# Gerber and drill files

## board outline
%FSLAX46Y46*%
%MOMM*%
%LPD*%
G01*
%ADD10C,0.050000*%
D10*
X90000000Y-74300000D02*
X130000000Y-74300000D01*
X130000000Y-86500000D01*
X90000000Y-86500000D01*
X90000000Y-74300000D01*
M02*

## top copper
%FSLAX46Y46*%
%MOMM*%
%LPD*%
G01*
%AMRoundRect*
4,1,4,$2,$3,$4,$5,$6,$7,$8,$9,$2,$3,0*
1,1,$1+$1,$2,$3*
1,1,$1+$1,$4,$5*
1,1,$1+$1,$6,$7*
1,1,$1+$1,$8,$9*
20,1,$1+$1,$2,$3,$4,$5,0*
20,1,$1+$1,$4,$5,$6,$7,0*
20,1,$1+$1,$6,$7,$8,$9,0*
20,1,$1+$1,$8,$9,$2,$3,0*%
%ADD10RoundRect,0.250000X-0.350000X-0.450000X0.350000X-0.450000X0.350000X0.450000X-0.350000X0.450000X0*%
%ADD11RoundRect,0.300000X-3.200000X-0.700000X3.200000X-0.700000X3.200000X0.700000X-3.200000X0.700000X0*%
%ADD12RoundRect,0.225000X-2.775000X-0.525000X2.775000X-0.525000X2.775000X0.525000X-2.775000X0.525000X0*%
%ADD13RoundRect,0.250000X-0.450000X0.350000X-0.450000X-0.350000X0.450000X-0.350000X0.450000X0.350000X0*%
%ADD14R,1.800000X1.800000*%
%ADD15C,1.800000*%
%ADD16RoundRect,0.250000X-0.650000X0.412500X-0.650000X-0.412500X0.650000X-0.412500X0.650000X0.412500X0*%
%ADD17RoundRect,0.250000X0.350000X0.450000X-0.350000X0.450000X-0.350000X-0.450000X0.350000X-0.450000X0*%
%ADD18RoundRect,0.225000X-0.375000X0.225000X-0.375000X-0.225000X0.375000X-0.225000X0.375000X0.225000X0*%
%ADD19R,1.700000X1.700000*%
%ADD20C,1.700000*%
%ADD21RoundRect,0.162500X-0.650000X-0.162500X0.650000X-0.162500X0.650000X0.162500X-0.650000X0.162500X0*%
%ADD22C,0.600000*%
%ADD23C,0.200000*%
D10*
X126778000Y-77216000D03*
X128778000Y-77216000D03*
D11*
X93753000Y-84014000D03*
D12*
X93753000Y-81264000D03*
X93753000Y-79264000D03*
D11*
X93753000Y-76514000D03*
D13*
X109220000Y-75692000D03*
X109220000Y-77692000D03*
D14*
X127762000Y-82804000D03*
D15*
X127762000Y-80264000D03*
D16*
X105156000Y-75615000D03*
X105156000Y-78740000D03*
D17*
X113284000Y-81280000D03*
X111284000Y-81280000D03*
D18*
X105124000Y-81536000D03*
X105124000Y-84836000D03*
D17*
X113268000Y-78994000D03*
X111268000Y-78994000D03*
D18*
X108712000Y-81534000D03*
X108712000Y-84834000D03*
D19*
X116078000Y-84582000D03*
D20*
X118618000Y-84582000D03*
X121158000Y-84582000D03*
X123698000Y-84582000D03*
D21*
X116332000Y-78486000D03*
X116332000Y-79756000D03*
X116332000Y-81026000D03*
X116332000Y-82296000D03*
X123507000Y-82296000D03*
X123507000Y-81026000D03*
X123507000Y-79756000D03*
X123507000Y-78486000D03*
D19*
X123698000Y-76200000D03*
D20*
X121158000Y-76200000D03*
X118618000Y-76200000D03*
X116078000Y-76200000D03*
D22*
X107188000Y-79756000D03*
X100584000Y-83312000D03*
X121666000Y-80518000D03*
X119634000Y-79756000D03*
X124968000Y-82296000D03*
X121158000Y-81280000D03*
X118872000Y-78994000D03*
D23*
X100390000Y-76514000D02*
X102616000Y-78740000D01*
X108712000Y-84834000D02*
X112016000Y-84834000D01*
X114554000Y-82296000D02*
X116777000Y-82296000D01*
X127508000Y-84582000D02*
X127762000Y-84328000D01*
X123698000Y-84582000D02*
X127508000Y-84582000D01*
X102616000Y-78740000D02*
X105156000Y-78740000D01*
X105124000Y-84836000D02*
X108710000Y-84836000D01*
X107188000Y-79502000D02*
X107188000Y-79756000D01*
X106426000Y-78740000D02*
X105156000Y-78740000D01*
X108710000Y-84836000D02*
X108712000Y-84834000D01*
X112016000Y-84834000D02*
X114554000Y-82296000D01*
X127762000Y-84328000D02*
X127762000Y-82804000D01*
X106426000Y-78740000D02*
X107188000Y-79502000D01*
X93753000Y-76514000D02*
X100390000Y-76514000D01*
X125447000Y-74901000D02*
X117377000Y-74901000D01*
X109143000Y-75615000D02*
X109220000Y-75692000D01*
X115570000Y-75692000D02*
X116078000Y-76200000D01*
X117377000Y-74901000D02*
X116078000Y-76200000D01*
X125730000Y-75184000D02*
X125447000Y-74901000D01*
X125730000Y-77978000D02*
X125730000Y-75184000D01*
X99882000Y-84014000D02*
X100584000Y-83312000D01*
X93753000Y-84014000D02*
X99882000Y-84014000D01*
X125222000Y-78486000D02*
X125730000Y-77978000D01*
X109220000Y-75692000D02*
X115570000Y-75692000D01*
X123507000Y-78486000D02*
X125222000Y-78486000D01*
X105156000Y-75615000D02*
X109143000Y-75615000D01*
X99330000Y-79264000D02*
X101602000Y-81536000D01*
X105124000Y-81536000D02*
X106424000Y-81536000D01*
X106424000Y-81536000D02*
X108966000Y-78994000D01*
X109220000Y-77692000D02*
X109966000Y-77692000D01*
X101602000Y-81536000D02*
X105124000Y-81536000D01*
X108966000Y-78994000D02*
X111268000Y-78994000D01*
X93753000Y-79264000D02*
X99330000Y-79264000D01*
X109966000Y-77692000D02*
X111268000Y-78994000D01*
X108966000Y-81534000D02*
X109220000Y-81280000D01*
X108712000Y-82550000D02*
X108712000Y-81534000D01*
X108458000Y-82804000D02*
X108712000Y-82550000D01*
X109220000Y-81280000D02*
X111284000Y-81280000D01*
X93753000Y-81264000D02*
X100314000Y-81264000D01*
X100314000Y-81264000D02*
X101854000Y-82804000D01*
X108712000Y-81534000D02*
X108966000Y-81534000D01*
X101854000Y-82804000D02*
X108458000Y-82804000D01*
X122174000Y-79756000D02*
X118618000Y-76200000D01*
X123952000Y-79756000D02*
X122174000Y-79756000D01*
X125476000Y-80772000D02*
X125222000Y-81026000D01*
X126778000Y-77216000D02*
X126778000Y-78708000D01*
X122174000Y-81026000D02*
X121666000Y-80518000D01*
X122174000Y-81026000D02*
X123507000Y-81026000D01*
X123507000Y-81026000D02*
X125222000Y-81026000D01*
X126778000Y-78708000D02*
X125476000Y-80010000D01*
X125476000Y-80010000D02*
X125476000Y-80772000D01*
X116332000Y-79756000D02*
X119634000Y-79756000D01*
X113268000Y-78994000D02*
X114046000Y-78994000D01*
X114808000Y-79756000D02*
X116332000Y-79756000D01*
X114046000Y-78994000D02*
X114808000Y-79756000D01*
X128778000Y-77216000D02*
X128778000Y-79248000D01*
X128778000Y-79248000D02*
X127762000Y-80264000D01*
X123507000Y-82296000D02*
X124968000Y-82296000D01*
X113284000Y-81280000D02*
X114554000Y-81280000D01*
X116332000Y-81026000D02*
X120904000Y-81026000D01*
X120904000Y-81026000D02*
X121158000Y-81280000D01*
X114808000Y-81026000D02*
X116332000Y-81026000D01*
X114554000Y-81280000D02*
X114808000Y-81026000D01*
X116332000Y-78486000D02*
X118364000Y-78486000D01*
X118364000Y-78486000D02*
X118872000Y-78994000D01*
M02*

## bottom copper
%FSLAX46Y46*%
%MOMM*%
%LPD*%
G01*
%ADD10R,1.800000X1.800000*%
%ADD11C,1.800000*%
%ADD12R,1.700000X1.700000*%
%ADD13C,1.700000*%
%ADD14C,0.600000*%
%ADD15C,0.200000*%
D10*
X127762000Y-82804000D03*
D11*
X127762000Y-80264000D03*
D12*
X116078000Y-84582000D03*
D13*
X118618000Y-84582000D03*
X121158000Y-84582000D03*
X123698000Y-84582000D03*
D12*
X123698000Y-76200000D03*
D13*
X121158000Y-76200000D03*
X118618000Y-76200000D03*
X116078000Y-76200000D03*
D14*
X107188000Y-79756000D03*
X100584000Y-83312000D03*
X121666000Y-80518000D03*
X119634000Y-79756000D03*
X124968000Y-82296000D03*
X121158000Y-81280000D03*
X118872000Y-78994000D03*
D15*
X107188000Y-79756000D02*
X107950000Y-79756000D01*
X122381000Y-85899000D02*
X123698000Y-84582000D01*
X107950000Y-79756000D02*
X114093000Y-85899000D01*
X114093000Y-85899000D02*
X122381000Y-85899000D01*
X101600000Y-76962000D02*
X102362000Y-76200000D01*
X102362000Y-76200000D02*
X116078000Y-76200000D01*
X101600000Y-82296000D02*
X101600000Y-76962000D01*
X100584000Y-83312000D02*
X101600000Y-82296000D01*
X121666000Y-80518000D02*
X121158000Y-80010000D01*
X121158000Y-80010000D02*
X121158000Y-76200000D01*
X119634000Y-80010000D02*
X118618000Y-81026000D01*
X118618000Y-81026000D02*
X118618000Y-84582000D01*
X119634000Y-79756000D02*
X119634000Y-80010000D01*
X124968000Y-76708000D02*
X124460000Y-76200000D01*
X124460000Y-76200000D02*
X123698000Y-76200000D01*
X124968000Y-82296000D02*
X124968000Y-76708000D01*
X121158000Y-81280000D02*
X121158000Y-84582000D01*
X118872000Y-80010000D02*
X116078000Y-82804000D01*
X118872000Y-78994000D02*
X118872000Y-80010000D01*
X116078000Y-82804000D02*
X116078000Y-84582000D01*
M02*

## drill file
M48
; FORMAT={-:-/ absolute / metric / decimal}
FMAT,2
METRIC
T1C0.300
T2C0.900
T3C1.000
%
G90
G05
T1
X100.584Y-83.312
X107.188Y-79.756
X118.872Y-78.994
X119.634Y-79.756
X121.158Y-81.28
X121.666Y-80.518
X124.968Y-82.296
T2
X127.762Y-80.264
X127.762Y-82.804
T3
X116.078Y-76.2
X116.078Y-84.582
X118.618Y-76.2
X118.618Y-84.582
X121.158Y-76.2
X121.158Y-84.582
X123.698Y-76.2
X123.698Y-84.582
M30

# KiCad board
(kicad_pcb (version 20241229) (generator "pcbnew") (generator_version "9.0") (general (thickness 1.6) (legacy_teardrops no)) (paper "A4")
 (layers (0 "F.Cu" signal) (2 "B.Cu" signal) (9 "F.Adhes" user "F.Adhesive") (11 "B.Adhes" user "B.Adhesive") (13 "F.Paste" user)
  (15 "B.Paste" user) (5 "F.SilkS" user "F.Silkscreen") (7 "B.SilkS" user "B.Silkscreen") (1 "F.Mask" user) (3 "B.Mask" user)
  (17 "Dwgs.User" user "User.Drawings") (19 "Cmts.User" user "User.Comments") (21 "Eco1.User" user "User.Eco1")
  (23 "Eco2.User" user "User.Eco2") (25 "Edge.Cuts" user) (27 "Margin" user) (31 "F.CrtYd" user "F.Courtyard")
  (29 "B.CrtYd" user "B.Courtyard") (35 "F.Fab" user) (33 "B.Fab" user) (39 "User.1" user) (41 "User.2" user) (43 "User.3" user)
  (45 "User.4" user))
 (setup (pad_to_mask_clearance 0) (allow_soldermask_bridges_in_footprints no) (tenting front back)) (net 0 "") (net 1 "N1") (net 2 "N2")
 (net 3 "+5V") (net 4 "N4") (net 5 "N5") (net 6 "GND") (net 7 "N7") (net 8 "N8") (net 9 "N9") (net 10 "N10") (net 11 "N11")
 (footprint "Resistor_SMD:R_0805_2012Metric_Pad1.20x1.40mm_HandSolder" (layer "F.Cu") (at 127.778 77.216)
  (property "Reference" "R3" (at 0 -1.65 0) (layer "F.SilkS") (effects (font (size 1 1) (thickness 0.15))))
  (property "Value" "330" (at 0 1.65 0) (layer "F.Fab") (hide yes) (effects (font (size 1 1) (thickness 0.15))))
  (pad "1" smd roundrect (at -1 0) (size 1.2 1.4) (layers "F.Cu" "F.Mask" "F.Paste") (roundrect_rratio 0.208333) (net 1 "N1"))
  (pad "2" smd roundrect (at 1 0) (size 1.2 1.4) (layers "F.Cu" "F.Mask" "F.Paste") (roundrect_rratio 0.208333) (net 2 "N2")))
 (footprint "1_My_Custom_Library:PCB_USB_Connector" (layer "F.Cu") (at 93.753 80.264)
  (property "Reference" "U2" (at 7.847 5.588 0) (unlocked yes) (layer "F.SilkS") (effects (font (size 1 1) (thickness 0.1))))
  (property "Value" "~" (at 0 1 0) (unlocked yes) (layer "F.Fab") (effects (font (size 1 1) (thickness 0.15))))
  (pad "1" smd roundrect (at 0 3.75) (size 7 2) (layers "F.Cu" "F.Mask" "F.Paste") (roundrect_rratio 0.15) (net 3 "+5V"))
  (pad "2" smd roundrect (at 0 1) (size 6 1.5) (layers "F.Cu" "F.Mask" "F.Paste") (roundrect_rratio 0.15) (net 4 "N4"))
  (pad "3" smd roundrect (at 0 -1) (size 6 1.5) (layers "F.Cu" "F.Mask" "F.Paste") (roundrect_rratio 0.15) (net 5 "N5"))
  (pad "4" smd roundrect (at 0 -3.75) (size 7 2) (layers "F.Cu" "F.Mask" "F.Paste") (roundrect_rratio 0.15) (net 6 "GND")))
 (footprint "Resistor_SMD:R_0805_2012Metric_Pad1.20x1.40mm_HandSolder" (layer "F.Cu") (at 109.22 76.692 -90)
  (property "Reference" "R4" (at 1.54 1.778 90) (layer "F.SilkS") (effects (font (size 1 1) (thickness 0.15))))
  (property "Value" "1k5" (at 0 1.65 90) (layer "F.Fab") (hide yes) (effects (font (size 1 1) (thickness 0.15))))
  (pad "1" smd roundrect (at -1 0 270) (size 1.2 1.4) (layers "F.Cu" "F.Mask" "F.Paste") (roundrect_rratio 0.208333) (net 3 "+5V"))
  (pad "2" smd roundrect (at 1 0 270) (size 1.2 1.4) (layers "F.Cu" "F.Mask" "F.Paste") (roundrect_rratio 0.208333) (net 5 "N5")))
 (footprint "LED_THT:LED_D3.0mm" (layer "F.Cu") (at 127.762 82.804 90)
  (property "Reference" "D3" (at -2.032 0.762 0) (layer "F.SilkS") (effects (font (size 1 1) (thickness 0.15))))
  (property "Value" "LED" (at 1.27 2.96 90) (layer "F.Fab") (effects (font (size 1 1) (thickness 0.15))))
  (pad "1" thru_hole rect (at 0 0 90) (size 1.8 1.8) (drill 0.9) (layers "*.Cu" "*.Mask") (remove_unused_layers no) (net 6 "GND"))
  (pad "2" thru_hole circle (at 2.54 0 90) (size 1.8 1.8) (drill 0.9) (layers "*.Cu" "*.Mask") (remove_unused_layers no) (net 2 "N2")))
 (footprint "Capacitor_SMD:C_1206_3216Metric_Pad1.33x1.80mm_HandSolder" (layer "F.Cu") (at 105.156 77.1775 -90)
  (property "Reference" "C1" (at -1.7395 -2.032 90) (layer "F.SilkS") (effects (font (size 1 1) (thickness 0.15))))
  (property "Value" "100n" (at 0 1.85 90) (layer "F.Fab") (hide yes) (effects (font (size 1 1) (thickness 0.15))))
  (pad "1" smd roundrect (at -1.5625 0 270) (size 1.325 1.8) (layers "F.Cu" "F.Mask" "F.Paste") (roundrect_rratio 0.188679) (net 3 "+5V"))
  (pad "2" smd roundrect (at 1.5625 0 270) (size 1.325 1.8) (layers "F.Cu" "F.Mask" "F.Paste") (roundrect_rratio 0.188679) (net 6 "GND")))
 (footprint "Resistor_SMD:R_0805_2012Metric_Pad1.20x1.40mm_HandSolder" (layer "F.Cu") (at 112.284 81.28 180)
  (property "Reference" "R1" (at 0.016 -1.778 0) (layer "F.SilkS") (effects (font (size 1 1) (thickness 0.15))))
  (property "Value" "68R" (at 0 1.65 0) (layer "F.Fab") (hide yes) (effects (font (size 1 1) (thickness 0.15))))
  (pad "1" smd roundrect (at -1 0 180) (size 1.2 1.4) (layers "F.Cu" "F.Mask" "F.Paste") (roundrect_rratio 0.208333) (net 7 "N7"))
  (pad "2" smd roundrect (at 1 0 180) (size 1.2 1.4) (layers "F.Cu" "F.Mask" "F.Paste") (roundrect_rratio 0.208333) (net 4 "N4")))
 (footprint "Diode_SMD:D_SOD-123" (layer "F.Cu") (at 105.124 83.186 -90)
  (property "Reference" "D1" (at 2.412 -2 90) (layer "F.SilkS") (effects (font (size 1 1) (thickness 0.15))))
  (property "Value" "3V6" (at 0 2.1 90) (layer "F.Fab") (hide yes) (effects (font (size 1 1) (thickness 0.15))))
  (pad "1" smd roundrect (at -1.65 0 270) (size 0.9 1.2) (layers "F.Cu" "F.Mask" "F.Paste") (roundrect_rratio 0.25) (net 5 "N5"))
  (pad "2" smd roundrect (at 1.65 0 270) (size 0.9 1.2) (layers "F.Cu" "F.Mask" "F.Paste") (roundrect_rratio 0.25) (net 6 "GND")))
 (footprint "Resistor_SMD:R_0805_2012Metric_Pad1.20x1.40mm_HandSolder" (layer "F.Cu") (at 112.268 78.994 180)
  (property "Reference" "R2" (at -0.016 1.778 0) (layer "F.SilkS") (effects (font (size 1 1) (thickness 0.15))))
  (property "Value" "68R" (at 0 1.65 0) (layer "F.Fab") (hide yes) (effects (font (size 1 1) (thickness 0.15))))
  (pad "1" smd roundrect (at -1 0 180) (size 1.2 1.4) (layers "F.Cu" "F.Mask" "F.Paste") (roundrect_rratio 0.208333) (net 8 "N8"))
  (pad "2" smd roundrect (at 1 0 180) (size 1.2 1.4) (layers "F.Cu" "F.Mask" "F.Paste") (roundrect_rratio 0.208333) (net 5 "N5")))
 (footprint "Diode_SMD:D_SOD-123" (layer "F.Cu") (at 108.712 83.184 -90)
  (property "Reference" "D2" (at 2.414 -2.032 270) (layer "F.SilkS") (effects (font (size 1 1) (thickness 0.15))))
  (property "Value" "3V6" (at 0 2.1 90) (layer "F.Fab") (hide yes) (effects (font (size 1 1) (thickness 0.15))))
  (pad "1" smd roundrect (at -1.65 0 270) (size 0.9 1.2) (layers "F.Cu" "F.Mask" "F.Paste") (roundrect_rratio 0.25) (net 4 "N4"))
  (pad "2" smd roundrect (at 1.65 0 270) (size 0.9 1.2) (layers "F.Cu" "F.Mask" "F.Paste") (roundrect_rratio 0.25) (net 6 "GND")))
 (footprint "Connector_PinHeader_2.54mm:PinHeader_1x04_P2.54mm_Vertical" (layer "F.Cu") (at 116.078 84.582 90)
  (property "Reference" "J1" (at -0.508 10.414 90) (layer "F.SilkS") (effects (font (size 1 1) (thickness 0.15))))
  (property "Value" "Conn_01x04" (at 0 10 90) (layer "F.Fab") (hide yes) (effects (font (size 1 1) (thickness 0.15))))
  (pad "1" thru_hole rect (at 0 0 90) (size 1.7 1.7) (drill 1) (layers "*.Cu" "*.Mask") (remove_unused_layers no) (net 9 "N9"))
  (pad "2" thru_hole circle (at 0 2.54 90) (size 1.7 1.7) (drill 1) (layers "*.Cu" "*.Mask") (remove_unused_layers no) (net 8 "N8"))
  (pad "3" thru_hole circle (at 0 5.08 90) (size 1.7 1.7) (drill 1) (layers "*.Cu" "*.Mask") (remove_unused_layers no) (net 7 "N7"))
  (pad "4" thru_hole circle (at 0 7.62 90) (size 1.7 1.7) (drill 1) (layers "*.Cu" "*.Mask") (remove_unused_layers no) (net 6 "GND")))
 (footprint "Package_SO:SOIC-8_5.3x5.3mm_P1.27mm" (layer "F.Cu") (at 119.9195 80.391)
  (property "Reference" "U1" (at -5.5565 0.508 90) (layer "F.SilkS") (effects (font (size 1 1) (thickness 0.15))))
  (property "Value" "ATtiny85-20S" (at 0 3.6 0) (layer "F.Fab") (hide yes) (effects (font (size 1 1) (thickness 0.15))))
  (pad "1" smd roundrect (at -3.5875 -1.905) (size 1.625 0.65) (layers "F.Cu" "F.Mask" "F.Paste") (roundrect_rratio 0.25) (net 9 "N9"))
  (pad "2" smd roundrect (at -3.5875 -0.635) (size 1.625 0.65) (layers "F.Cu" "F.Mask" "F.Paste") (roundrect_rratio 0.25) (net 8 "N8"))
  (pad "3" smd roundrect (at -3.5875 0.635) (size 1.625 0.65) (layers "F.Cu" "F.Mask" "F.Paste") (roundrect_rratio 0.25) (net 7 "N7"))
  (pad "4" smd roundrect (at -3.5875 1.905) (size 1.625 0.65) (layers "F.Cu" "F.Mask" "F.Paste") (roundrect_rratio 0.25) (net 6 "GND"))
  (pad "5" smd roundrect (at 3.5875 1.905) (size 1.625 0.65) (layers "F.Cu" "F.Mask" "F.Paste") (roundrect_rratio 0.25) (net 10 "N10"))
  (pad "6" smd roundrect (at 3.5875 0.635) (size 1.625 0.65) (layers "F.Cu" "F.Mask" "F.Paste") (roundrect_rratio 0.25) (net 1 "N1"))
  (pad "7" smd roundrect (at 3.5875 -0.635) (size 1.625 0.65) (layers "F.Cu" "F.Mask" "F.Paste") (roundrect_rratio 0.25) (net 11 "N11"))
  (pad "8" smd roundrect (at 3.5875 -1.905) (size 1.625 0.65) (layers "F.Cu" "F.Mask" "F.Paste") (roundrect_rratio 0.25) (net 3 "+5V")))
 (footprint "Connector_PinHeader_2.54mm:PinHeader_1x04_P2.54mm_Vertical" (layer "F.Cu") (at 123.698 76.2 -90)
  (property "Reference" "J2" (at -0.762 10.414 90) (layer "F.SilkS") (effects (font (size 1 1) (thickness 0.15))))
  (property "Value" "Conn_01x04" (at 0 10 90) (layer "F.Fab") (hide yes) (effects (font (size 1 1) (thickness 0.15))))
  (pad "1" thru_hole rect (at 0 0 270) (size 1.7 1.7) (drill 1) (layers "*.Cu" "*.Mask") (remove_unused_layers no) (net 10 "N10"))
  (pad "2" thru_hole circle (at 0 2.54 270) (size 1.7 1.7) (drill 1) (layers "*.Cu" "*.Mask") (remove_unused_layers no) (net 1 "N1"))
  (pad "3" thru_hole circle (at 0 5.08 270) (size 1.7 1.7) (drill 1) (layers "*.Cu" "*.Mask") (remove_unused_layers no) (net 11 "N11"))
  (pad "4" thru_hole circle (at 0 7.62 270) (size 1.7 1.7) (drill 1) (layers "*.Cu" "*.Mask") (remove_unused_layers no) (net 3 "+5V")))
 (gr_rect (start 90 74.3) (end 130 86.5) (stroke (width 0.05) (type solid)) (fill no) (layer "Edge.Cuts"))
 (segment (start 100.39 76.514) (end 102.616 78.74) (width 0.2) (layer "F.Cu") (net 6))
 (segment (start 108.712 84.834) (end 112.016 84.834) (width 0.2) (layer "F.Cu") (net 6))
 (segment (start 114.554 82.296) (end 116.777 82.296) (width 0.2) (layer "F.Cu") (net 6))
 (segment (start 127.508 84.582) (end 127.762 84.328) (width 0.2) (layer "F.Cu") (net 6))
 (segment (start 123.698 84.582) (end 127.508 84.582) (width 0.2) (layer "F.Cu") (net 6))
 (segment (start 102.616 78.74) (end 105.156 78.74) (width 0.2) (layer "F.Cu") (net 6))
 (segment (start 105.124 84.836) (end 108.71 84.836) (width 0.2) (layer "F.Cu") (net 6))
 (segment (start 107.188 79.502) (end 107.188 79.756) (width 0.2) (layer "F.Cu") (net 6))
 (segment (start 106.426 78.74) (end 105.156 78.74) (width 0.2) (layer "F.Cu") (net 6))
 (segment (start 108.71 84.836) (end 108.712 84.834) (width 0.2) (layer "F.Cu") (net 6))
 (segment (start 112.016 84.834) (end 114.554 82.296) (width 0.2) (layer "F.Cu") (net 6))
 (segment (start 127.762 84.328) (end 127.762 82.804) (width 0.2) (layer "F.Cu") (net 6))
 (segment (start 106.426 78.74) (end 107.188 79.502) (width 0.2) (layer "F.Cu") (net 6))
 (segment (start 93.753 76.514) (end 100.39 76.514) (width 0.2) (layer "F.Cu") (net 6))
 (via (at 107.188 79.756) (size 0.6) (drill 0.3) (layers "F.Cu" "B.Cu") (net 6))
 (segment (start 107.188 79.756) (end 107.95 79.756) (width 0.2) (layer "B.Cu") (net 6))
 (segment (start 122.381 85.899) (end 123.698 84.582) (width 0.2) (layer "B.Cu") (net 6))
 (segment (start 107.95 79.756) (end 114.093 85.899) (width 0.2) (layer "B.Cu") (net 6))
 (segment (start 114.093 85.899) (end 122.381 85.899) (width 0.2) (layer "B.Cu") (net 6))
 (segment (start 125.447 74.901) (end 117.377 74.901) (width 0.2) (layer "F.Cu") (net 3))
 (segment (start 109.143 75.615) (end 109.22 75.692) (width 0.2) (layer "F.Cu") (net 3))
 (segment (start 115.57 75.692) (end 116.078 76.2) (width 0.2) (layer "F.Cu") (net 3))
 (segment (start 117.377 74.901) (end 116.078 76.2) (width 0.2) (layer "F.Cu") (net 3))
 (segment (start 125.73 75.184) (end 125.447 74.901) (width 0.2) (layer "F.Cu") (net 3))
 (segment (start 125.73 77.978) (end 125.73 75.184) (width 0.2) (layer "F.Cu") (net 3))
 (segment (start 99.882 84.014) (end 100.584 83.312) (width 0.2) (layer "F.Cu") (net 3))
 (segment (start 93.753 84.014) (end 99.882 84.014) (width 0.2) (layer "F.Cu") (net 3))
 (segment (start 125.222 78.486) (end 125.73 77.978) (width 0.2) (layer "F.Cu") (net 3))
 (segment (start 109.22 75.692) (end 115.57 75.692) (width 0.2) (layer "F.Cu") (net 3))
 (segment (start 123.507 78.486) (end 125.222 78.486) (width 0.2) (layer "F.Cu") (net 3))
 (segment (start 105.156 75.615) (end 109.143 75.615) (width 0.2) (layer "F.Cu") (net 3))
 (via (at 100.584 83.312) (size 0.6) (drill 0.3) (layers "F.Cu" "B.Cu") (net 3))
 (segment (start 101.6 76.962) (end 102.362 76.2) (width 0.2) (layer "B.Cu") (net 3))
 (segment (start 102.362 76.2) (end 116.078 76.2) (width 0.2) (layer "B.Cu") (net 3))
 (segment (start 101.6 82.296) (end 101.6 76.962) (width 0.2) (layer "B.Cu") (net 3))
 (segment (start 100.584 83.312) (end 101.6 82.296) (width 0.2) (layer "B.Cu") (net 3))
 (segment (start 99.33 79.264) (end 101.602 81.536) (width 0.2) (layer "F.Cu") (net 5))
 (segment (start 105.124 81.536) (end 106.424 81.536) (width 0.2) (layer "F.Cu") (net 5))
 (segment (start 106.424 81.536) (end 108.966 78.994) (width 0.2) (layer "F.Cu") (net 5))
 (segment (start 109.22 77.692) (end 109.966 77.692) (width 0.2) (layer "F.Cu") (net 5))
 (segment (start 101.602 81.536) (end 105.124 81.536) (width 0.2) (layer "F.Cu") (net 5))
 (segment (start 108.966 78.994) (end 111.268 78.994) (width 0.2) (layer "F.Cu") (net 5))
 (segment (start 93.753 79.264) (end 99.33 79.264) (width 0.2) (layer "F.Cu") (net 5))
 (segment (start 109.966 77.692) (end 111.268 78.994) (width 0.2) (layer "F.Cu") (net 5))
 (segment (start 108.966 81.534) (end 109.22 81.28) (width 0.2) (layer "F.Cu") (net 4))
 (segment (start 108.712 82.55) (end 108.712 81.534) (width 0.2) (layer "F.Cu") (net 4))
 (segment (start 108.458 82.804) (end 108.712 82.55) (width 0.2) (layer "F.Cu") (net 4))
 (segment (start 109.22 81.28) (end 111.284 81.28) (width 0.2) (layer "F.Cu") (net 4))
 (segment (start 93.753 81.264) (end 100.314 81.264) (width 0.2) (layer "F.Cu") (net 4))
 (segment (start 100.314 81.264) (end 101.854 82.804) (width 0.2) (layer "F.Cu") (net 4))
 (segment (start 108.712 81.534) (end 108.966 81.534) (width 0.2) (layer "F.Cu") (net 4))
 (segment (start 101.854 82.804) (end 108.458 82.804) (width 0.2) (layer "F.Cu") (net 4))
 (segment (start 122.174 79.756) (end 118.618 76.2) (width 0.2) (layer "F.Cu") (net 11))
 (segment (start 123.952 79.756) (end 122.174 79.756) (width 0.2) (layer "F.Cu") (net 11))
 (segment (start 125.476 80.772) (end 125.222 81.026) (width 0.2) (layer "F.Cu") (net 1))
 (segment (start 126.778 77.216) (end 126.778 78.708) (width 0.2) (layer "F.Cu") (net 1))
 (segment (start 122.174 81.026) (end 121.666 80.518) (width 0.2) (layer "F.Cu") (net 1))
 (segment (start 122.174 81.026) (end 123.507 81.026) (width 0.2) (layer "F.Cu") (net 1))
 (segment (start 123.507 81.026) (end 125.222 81.026) (width 0.2) (layer "F.Cu") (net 1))
 (segment (start 126.778 78.708) (end 125.476 80.01) (width 0.2) (layer "F.Cu") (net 1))
 (segment (start 125.476 80.01) (end 125.476 80.772) (width 0.2) (layer "F.Cu") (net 1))
 (via (at 121.666 80.518) (size 0.6) (drill 0.3) (layers "F.Cu" "B.Cu") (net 1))
 (segment (start 121.666 80.518) (end 121.158 80.01) (width 0.2) (layer "B.Cu") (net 1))
 (segment (start 121.158 80.01) (end 121.158 76.2) (width 0.2) (layer "B.Cu") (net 1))
 (segment (start 116.332 79.756) (end 119.634 79.756) (width 0.2) (layer "F.Cu") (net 8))
 (segment (start 113.268 78.994) (end 114.046 78.994) (width 0.2) (layer "F.Cu") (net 8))
 (segment (start 114.808 79.756) (end 116.332 79.756) (width 0.2) (layer "F.Cu") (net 8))
 (segment (start 114.046 78.994) (end 114.808 79.756) (width 0.2) (layer "F.Cu") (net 8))
 (via (at 119.634 79.756) (size 0.6) (drill 0.3) (layers "F.Cu" "B.Cu") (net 8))
 (segment (start 119.634 80.01) (end 118.618 81.026) (width 0.2) (layer "B.Cu") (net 8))
 (segment (start 118.618 81.026) (end 118.618 84.582) (width 0.2) (layer "B.Cu") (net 8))
 (segment (start 119.634 79.756) (end 119.634 80.01) (width 0.2) (layer "B.Cu") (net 8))
 (segment (start 128.778 77.216) (end 128.778 79.248) (width 0.2) (layer "F.Cu") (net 2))
 (segment (start 128.778 79.248) (end 127.762 80.264) (width 0.2) (layer "F.Cu") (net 2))
 (segment (start 123.507 82.296) (end 124.968 82.296) (width 0.2) (layer "F.Cu") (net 10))
 (via (at 124.968 82.296) (size 0.6) (drill 0.3) (layers "F.Cu" "B.Cu") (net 10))
 (segment (start 124.968 76.708) (end 124.46 76.2) (width 0.2) (layer "B.Cu") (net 10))
 (segment (start 124.46 76.2) (end 123.698 76.2) (width 0.2) (layer "B.Cu") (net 10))
 (segment (start 124.968 82.296) (end 124.968 76.708) (width 0.2) (layer "B.Cu") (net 10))
 (segment (start 113.284 81.28) (end 114.554 81.28) (width 0.2) (layer "F.Cu") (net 7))
 (segment (start 116.332 81.026) (end 120.904 81.026) (width 0.2) (layer "F.Cu") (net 7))
 (segment (start 120.904 81.026) (end 121.158 81.28) (width 0.2) (layer "F.Cu") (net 7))
 (segment (start 114.808 81.026) (end 116.332 81.026) (width 0.2) (layer "F.Cu") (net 7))
 (segment (start 114.554 81.28) (end 114.808 81.026) (width 0.2) (layer "F.Cu") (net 7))
 (via (at 121.158 81.28) (size 0.6) (drill 0.3) (layers "F.Cu" "B.Cu") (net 7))
 (segment (start 121.158 81.28) (end 121.158 84.582) (width 0.2) (layer "B.Cu") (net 7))
 (segment (start 116.332 78.486) (end 118.364 78.486) (width 0.2) (layer "F.Cu") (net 9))
 (segment (start 118.364 78.486) (end 118.872 78.994) (width 0.2) (layer "F.Cu") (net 9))
 (via (at 118.872 78.994) (size 0.6) (drill 0.3) (layers "F.Cu" "B.Cu") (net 9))
 (segment (start 118.872 80.01) (end 116.078 82.804) (width 0.2) (layer "B.Cu") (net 9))
 (segment (start 118.872 78.994) (end 118.872 80.01) (width 0.2) (layer "B.Cu") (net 9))
 (segment (start 116.078 82.804) (end 116.078 84.582) (width 0.2) (layer "B.Cu") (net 9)))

